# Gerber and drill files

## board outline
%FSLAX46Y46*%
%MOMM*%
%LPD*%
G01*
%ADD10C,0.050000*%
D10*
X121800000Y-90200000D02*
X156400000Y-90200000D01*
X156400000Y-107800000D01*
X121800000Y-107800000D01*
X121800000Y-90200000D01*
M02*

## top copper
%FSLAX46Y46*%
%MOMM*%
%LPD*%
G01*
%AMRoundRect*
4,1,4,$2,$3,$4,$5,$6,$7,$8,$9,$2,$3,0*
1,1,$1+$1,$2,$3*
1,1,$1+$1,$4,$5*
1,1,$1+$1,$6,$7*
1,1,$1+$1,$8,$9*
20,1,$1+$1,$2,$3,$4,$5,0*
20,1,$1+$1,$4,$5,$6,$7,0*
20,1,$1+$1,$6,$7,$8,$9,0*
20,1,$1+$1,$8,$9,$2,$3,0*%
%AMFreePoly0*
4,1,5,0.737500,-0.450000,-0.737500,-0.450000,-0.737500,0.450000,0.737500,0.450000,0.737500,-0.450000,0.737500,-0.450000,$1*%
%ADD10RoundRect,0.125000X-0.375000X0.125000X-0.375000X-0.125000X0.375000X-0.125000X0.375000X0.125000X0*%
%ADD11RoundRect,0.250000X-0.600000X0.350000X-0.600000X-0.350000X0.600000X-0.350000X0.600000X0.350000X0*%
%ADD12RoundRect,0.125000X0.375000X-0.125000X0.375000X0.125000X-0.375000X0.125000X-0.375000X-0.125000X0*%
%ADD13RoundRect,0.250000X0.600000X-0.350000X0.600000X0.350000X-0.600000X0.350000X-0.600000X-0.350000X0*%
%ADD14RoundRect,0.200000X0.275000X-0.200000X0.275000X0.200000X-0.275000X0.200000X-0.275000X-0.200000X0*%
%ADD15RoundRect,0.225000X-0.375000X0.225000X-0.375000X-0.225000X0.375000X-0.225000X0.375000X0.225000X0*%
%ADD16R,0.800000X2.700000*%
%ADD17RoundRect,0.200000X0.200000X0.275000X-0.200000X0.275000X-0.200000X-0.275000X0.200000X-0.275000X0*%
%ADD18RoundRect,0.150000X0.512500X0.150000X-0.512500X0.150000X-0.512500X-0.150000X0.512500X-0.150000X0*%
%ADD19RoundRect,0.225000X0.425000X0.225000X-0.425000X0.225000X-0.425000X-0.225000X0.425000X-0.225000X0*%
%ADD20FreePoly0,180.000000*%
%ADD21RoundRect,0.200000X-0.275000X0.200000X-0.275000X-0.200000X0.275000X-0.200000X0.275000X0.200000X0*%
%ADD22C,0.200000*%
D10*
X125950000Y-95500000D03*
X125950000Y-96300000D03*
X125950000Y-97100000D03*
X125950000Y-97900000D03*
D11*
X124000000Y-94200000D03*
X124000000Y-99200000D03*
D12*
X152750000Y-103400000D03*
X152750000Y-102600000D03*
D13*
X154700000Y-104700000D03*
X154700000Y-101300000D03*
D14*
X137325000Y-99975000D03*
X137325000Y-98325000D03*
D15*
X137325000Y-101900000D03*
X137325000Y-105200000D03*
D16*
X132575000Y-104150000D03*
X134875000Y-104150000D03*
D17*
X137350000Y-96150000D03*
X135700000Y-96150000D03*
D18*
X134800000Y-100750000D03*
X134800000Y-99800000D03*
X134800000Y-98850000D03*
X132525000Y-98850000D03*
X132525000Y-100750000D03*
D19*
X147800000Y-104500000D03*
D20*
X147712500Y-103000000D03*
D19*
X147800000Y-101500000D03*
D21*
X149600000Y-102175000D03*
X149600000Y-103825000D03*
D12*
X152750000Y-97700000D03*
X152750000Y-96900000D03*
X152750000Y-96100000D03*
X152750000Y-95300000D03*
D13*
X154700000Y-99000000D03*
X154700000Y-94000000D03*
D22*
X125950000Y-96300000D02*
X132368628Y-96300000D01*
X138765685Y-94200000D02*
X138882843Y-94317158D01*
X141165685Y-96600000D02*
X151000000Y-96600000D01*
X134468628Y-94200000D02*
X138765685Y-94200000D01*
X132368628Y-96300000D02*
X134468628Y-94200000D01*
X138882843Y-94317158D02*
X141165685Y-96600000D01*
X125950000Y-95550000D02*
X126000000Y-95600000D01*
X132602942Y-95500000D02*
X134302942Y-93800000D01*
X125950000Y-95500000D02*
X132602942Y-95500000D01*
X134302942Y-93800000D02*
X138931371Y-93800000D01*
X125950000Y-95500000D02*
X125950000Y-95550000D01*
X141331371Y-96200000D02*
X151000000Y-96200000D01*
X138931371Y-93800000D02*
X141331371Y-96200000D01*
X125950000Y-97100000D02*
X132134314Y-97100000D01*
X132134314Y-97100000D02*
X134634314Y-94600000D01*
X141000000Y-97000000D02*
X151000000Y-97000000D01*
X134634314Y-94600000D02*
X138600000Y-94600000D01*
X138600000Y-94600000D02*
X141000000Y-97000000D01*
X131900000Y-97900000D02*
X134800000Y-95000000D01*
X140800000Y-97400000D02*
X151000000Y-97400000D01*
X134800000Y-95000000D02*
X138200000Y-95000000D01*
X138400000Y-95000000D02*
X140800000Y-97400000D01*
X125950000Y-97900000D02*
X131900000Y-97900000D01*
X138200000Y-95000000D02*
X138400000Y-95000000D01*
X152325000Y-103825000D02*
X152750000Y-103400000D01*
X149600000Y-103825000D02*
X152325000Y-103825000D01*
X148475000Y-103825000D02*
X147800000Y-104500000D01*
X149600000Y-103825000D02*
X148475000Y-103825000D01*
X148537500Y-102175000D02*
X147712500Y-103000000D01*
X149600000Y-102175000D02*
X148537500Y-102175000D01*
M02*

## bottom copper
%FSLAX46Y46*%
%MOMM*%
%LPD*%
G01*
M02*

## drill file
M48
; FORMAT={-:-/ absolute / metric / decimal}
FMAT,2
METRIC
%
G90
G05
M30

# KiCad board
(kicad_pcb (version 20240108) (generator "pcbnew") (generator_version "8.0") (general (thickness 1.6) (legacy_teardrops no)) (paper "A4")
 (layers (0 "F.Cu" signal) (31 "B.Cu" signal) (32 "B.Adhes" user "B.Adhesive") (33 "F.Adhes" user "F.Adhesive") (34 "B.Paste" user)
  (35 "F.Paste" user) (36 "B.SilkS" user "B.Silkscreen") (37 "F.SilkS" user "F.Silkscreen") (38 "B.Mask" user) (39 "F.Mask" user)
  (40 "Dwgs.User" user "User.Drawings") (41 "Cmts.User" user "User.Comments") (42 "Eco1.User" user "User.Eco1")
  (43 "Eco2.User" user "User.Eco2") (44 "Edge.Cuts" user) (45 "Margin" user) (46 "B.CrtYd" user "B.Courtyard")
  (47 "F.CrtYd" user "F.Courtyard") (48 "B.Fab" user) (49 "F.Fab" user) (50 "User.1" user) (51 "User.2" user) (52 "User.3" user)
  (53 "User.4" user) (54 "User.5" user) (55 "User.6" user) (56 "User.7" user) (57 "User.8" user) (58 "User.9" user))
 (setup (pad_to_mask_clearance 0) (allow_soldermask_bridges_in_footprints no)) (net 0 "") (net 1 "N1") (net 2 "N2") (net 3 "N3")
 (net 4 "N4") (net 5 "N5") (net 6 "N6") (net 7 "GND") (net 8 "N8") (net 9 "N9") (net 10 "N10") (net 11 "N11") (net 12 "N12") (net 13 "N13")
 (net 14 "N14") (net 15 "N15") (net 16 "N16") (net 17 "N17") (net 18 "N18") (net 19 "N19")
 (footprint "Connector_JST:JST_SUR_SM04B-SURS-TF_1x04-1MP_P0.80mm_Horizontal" (layer "F.Cu") (at 124.8 96.7 -90)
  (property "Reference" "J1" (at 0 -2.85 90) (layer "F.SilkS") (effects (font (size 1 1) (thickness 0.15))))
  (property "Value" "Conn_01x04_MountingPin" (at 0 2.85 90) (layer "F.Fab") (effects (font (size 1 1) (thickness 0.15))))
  (pad "1" smd roundrect (at -1.2 -1.15 270) (size 0.5 1) (layers "F.Cu" "F.Paste" "F.Mask") (roundrect_rratio 0.25) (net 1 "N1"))
  (pad "2" smd roundrect (at -0.4 -1.15 270) (size 0.5 1) (layers "F.Cu" "F.Paste" "F.Mask") (roundrect_rratio 0.25) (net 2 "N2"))
  (pad "3" smd roundrect (at 0.4 -1.15 270) (size 0.5 1) (layers "F.Cu" "F.Paste" "F.Mask") (roundrect_rratio 0.25) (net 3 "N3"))
  (pad "4" smd roundrect (at 1.2 -1.15 270) (size 0.5 1) (layers "F.Cu" "F.Paste" "F.Mask") (roundrect_rratio 0.25) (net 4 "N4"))
  (pad "MP" smd roundrect (at -2.5 0.8 270) (size 1.2 1.7) (layers "F.Cu" "F.Paste" "F.Mask") (roundrect_rratio 0.208333) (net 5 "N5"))
  (pad "MP" smd roundrect (at 2.5 0.8 270) (size 1.2 1.7) (layers "F.Cu" "F.Paste" "F.Mask") (roundrect_rratio 0.208333) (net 5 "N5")))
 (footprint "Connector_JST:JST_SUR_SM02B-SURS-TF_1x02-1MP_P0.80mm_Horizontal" (layer "F.Cu") (at 153.9 103 90)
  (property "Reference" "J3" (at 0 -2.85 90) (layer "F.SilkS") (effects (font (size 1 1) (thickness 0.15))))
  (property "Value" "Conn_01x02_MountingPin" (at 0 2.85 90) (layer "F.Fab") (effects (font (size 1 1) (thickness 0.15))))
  (pad "1" smd roundrect (at -0.4 -1.15 90) (size 0.5 1) (layers "F.Cu" "F.Paste" "F.Mask") (roundrect_rratio 0.25) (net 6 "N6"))
  (pad "2" smd roundrect (at 0.4 -1.15 90) (size 0.5 1) (layers "F.Cu" "F.Paste" "F.Mask") (roundrect_rratio 0.25) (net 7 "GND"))
  (pad "MP" smd roundrect (at -1.7 0.8 90) (size 1.2 1.7) (layers "F.Cu" "F.Paste" "F.Mask") (roundrect_rratio 0.208333) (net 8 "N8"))
  (pad "MP" smd roundrect (at 1.7 0.8 90) (size 1.2 1.7) (layers "F.Cu" "F.Paste" "F.Mask") (roundrect_rratio 0.208333) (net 8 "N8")))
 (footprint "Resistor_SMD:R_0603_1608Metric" (layer "F.Cu") (at 137.325 99.15 90)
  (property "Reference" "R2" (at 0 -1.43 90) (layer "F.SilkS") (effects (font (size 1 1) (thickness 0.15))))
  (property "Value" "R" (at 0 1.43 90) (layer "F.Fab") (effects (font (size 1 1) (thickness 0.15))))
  (pad "1" smd roundrect (at -0.825 0 90) (size 0.8 0.95) (layers "F.Cu" "F.Paste" "F.Mask") (roundrect_rratio 0.25) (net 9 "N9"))
  (pad "2" smd roundrect (at 0.825 0 90) (size 0.8 0.95) (layers "F.Cu" "F.Paste" "F.Mask") (roundrect_rratio 0.25) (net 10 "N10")))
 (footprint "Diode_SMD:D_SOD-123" (layer "F.Cu") (at 137.325 103.55 -90)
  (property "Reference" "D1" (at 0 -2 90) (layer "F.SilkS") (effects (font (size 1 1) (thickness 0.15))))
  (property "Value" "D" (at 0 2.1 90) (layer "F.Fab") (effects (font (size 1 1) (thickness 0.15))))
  (pad "1" smd roundrect (at -1.65 0 270) (size 0.9 1.2) (layers "F.Cu" "F.Paste" "F.Mask") (roundrect_rratio 0.25) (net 9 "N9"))
  (pad "2" smd roundrect (at 1.65 0 270) (size 0.9 1.2) (layers "F.Cu" "F.Paste" "F.Mask") (roundrect_rratio 0.25) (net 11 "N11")))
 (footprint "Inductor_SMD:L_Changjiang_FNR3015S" (layer "F.Cu") (at 133.725 104.15)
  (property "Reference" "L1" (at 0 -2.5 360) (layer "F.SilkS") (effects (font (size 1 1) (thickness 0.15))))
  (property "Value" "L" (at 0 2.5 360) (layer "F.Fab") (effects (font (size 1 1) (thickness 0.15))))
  (pad "1" smd rect (at -1.15 0) (size 0.8 2.7) (layers "F.Cu" "F.Paste" "F.Mask") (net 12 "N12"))
  (pad "2" smd rect (at 1.15 0) (size 0.8 2.7) (layers "F.Cu" "F.Paste" "F.Mask") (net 11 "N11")))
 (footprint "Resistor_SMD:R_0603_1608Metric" (layer "F.Cu") (at 136.525 96.15 180)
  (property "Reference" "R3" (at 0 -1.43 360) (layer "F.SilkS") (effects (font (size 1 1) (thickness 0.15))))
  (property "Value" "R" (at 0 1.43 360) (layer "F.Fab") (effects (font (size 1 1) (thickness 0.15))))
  (pad "1" smd roundrect (at -0.825 0 180) (size 0.8 0.95) (layers "F.Cu" "F.Paste" "F.Mask") (roundrect_rratio 0.25) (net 10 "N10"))
  (pad "2" smd roundrect (at 0.825 0 180) (size 0.8 0.95) (layers "F.Cu" "F.Paste" "F.Mask") (roundrect_rratio 0.25) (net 7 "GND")))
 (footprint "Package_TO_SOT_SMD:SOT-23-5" (layer "F.Cu") (at 133.6625 99.8 180)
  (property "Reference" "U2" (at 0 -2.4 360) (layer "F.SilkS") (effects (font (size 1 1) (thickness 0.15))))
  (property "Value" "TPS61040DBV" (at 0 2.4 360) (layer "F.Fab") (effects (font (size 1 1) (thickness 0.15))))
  (pad "1" smd roundrect (at -1.1375 -0.95 180) (size 1.325 0.6) (layers "F.Cu" "F.Paste" "F.Mask") (roundrect_rratio 0.25) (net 11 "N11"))
  (pad "2" smd roundrect (at -1.1375 0 180) (size 1.325 0.6) (layers "F.Cu" "F.Paste" "F.Mask") (roundrect_rratio 0.25) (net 7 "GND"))
  (pad "3" smd roundrect (at -1.1375 0.95 180) (size 1.325 0.6) (layers "F.Cu" "F.Paste" "F.Mask") (roundrect_rratio 0.25) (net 10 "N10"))
  (pad "4" smd roundrect (at 1.1375 0.95 180) (size 1.325 0.6) (layers "F.Cu" "F.Paste" "F.Mask") (roundrect_rratio 0.25) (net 12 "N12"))
  (pad "5" smd roundrect (at 1.1375 -0.95 180) (size 1.325 0.6) (layers "F.Cu" "F.Paste" "F.Mask") (roundrect_rratio 0.25) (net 12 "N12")))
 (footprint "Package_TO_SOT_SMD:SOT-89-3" (layer "F.Cu") (at 145.85 103 180)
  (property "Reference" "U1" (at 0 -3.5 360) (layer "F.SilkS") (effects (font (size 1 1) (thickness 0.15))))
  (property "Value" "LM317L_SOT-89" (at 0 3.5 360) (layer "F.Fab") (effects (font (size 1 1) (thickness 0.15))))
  (pad "1" smd roundrect (at -1.95 -1.5 180) (size 1.3 0.9) (layers "F.Cu" "F.Paste" "F.Mask") (roundrect_rratio 0.25) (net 6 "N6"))
  (pad "2" smd custom (at -1.8625 0 180) (size 1.475 0.9) (layers "F.Cu" "F.Paste" "F.Mask") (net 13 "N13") (zone_connect 2)
   (thermal_bridge_angle 45) (options (clearance outline) (anchor rect)) (primitives))
  (pad "3" smd roundrect (at -1.95 1.5 180) (size 1.3 0.9) (layers "F.Cu" "F.Paste" "F.Mask") (roundrect_rratio 0.25) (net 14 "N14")))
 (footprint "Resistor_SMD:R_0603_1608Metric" (layer "F.Cu") (at 149.6 103 -90)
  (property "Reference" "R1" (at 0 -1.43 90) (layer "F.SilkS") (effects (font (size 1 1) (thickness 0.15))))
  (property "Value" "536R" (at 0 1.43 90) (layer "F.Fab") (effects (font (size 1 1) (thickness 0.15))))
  (pad "1" smd roundrect (at -0.825 0 270) (size 0.8 0.95) (layers "F.Cu" "F.Paste" "F.Mask") (roundrect_rratio 0.25) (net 13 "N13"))
  (pad "2" smd roundrect (at 0.825 0 270) (size 0.8 0.95) (layers "F.Cu" "F.Paste" "F.Mask") (roundrect_rratio 0.25) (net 6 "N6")))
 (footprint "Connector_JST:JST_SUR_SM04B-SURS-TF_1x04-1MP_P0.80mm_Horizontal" (layer "F.Cu") (at 153.9 96.5 90)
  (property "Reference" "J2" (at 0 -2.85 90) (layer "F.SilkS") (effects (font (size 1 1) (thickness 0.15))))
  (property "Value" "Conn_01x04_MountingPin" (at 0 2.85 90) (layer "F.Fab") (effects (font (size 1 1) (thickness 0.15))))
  (pad "1" smd roundrect (at -1.2 -1.15 90) (size 0.5 1) (layers "F.Cu" "F.Paste" "F.Mask") (roundrect_rratio 0.25) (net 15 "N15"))
  (pad "2" smd roundrect (at -0.4 -1.15 90) (size 0.5 1) (layers "F.Cu" "F.Paste" "F.Mask") (roundrect_rratio 0.25) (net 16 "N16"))
  (pad "3" smd roundrect (at 0.4 -1.15 90) (size 0.5 1) (layers "F.Cu" "F.Paste" "F.Mask") (roundrect_rratio 0.25) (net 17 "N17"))
  (pad "4" smd roundrect (at 1.2 -1.15 90) (size 0.5 1) (layers "F.Cu" "F.Paste" "F.Mask") (roundrect_rratio 0.25) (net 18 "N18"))
  (pad "MP" smd roundrect (at -2.5 0.8 90) (size 1.2 1.7) (layers "F.Cu" "F.Paste" "F.Mask") (roundrect_rratio 0.208333) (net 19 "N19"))
  (pad "MP" smd roundrect (at 2.5 0.8 90) (size 1.2 1.7) (layers "F.Cu" "F.Paste" "F.Mask") (roundrect_rratio 0.208333) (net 19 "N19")))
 (gr_rect (start 121.8 90.2) (end 156.4 107.8) (stroke (width 0.05) (type default)) (fill none) (layer "Edge.Cuts"))
 (segment (start 125.95 96.3) (end 132.368628 96.3) (width 0.2) (layer "F.Cu") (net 2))
 (segment (start 138.765685 94.2) (end 138.882843 94.317158) (width 0.2) (layer "F.Cu") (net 2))
 (segment (start 141.165685 96.6) (end 151 96.6) (width 0.2) (layer "F.Cu") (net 2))
 (segment (start 134.468628 94.2) (end 138.765685 94.2) (width 0.2) (layer "F.Cu") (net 2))
 (segment (start 132.368628 96.3) (end 134.468628 94.2) (width 0.2) (layer "F.Cu") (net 2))
 (segment (start 138.882843 94.317158) (end 141.165685 96.6) (width 0.2) (layer "F.Cu") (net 2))
 (segment (start 125.95 95.55) (end 126 95.6) (width 0.2) (layer "F.Cu") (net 1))
 (segment (start 132.602942 95.5) (end 134.302942 93.8) (width 0.2) (layer "F.Cu") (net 1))
 (segment (start 125.95 95.5) (end 132.602942 95.5) (width 0.2) (layer "F.Cu") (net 1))
 (segment (start 134.302942 93.8) (end 138.931371 93.8) (width 0.2) (layer "F.Cu") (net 1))
 (segment (start 125.95 95.5) (end 125.95 95.55) (width 0.2) (layer "F.Cu") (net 1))
 (segment (start 141.331371 96.2) (end 151 96.2) (width 0.2) (layer "F.Cu") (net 1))
 (segment (start 138.931371 93.8) (end 141.331371 96.2) (width 0.2) (layer "F.Cu") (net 1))
 (segment (start 125.95 97.1) (end 132.134314 97.1) (width 0.2) (layer "F.Cu") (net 3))
 (segment (start 132.134314 97.1) (end 134.634314 94.6) (width 0.2) (layer "F.Cu") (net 3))
 (segment (start 141 97) (end 151 97) (width 0.2) (layer "F.Cu") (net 3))
 (segment (start 134.634314 94.6) (end 138.6 94.6) (width 0.2) (layer "F.Cu") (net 3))
 (segment (start 138.6 94.6) (end 141 97) (width 0.2) (layer "F.Cu") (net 3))
 (segment (start 131.9 97.9) (end 134.8 95) (width 0.2) (layer "F.Cu") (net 4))
 (segment (start 140.8 97.4) (end 151 97.4) (width 0.2) (layer "F.Cu") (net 4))
 (segment (start 134.8 95) (end 138.2 95) (width 0.2) (layer "F.Cu") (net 4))
 (segment (start 138.4 95) (end 140.8 97.4) (width 0.2) (layer "F.Cu") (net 4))
 (segment (start 125.95 97.9) (end 131.9 97.9) (width 0.2) (layer "F.Cu") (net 4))
 (segment (start 138.2 95) (end 138.4 95) (width 0.2) (layer "F.Cu") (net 4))
 (segment (start 152.325 103.825) (end 152.75 103.4) (width 0.2) (layer "F.Cu") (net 6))
 (segment (start 149.6 103.825) (end 152.325 103.825) (width 0.2) (layer "F.Cu") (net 6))
 (segment (start 148.475 103.825) (end 147.8 104.5) (width 0.2) (layer "F.Cu") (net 6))
 (segment (start 149.6 103.825) (end 148.475 103.825) (width 0.2) (layer "F.Cu") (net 6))
 (segment (start 148.5375 102.175) (end 147.7125 103) (width 0.2) (layer "F.Cu") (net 13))
 (segment (start 149.6 102.175) (end 148.5375 102.175) (width 0.2) (layer "F.Cu") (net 13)))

